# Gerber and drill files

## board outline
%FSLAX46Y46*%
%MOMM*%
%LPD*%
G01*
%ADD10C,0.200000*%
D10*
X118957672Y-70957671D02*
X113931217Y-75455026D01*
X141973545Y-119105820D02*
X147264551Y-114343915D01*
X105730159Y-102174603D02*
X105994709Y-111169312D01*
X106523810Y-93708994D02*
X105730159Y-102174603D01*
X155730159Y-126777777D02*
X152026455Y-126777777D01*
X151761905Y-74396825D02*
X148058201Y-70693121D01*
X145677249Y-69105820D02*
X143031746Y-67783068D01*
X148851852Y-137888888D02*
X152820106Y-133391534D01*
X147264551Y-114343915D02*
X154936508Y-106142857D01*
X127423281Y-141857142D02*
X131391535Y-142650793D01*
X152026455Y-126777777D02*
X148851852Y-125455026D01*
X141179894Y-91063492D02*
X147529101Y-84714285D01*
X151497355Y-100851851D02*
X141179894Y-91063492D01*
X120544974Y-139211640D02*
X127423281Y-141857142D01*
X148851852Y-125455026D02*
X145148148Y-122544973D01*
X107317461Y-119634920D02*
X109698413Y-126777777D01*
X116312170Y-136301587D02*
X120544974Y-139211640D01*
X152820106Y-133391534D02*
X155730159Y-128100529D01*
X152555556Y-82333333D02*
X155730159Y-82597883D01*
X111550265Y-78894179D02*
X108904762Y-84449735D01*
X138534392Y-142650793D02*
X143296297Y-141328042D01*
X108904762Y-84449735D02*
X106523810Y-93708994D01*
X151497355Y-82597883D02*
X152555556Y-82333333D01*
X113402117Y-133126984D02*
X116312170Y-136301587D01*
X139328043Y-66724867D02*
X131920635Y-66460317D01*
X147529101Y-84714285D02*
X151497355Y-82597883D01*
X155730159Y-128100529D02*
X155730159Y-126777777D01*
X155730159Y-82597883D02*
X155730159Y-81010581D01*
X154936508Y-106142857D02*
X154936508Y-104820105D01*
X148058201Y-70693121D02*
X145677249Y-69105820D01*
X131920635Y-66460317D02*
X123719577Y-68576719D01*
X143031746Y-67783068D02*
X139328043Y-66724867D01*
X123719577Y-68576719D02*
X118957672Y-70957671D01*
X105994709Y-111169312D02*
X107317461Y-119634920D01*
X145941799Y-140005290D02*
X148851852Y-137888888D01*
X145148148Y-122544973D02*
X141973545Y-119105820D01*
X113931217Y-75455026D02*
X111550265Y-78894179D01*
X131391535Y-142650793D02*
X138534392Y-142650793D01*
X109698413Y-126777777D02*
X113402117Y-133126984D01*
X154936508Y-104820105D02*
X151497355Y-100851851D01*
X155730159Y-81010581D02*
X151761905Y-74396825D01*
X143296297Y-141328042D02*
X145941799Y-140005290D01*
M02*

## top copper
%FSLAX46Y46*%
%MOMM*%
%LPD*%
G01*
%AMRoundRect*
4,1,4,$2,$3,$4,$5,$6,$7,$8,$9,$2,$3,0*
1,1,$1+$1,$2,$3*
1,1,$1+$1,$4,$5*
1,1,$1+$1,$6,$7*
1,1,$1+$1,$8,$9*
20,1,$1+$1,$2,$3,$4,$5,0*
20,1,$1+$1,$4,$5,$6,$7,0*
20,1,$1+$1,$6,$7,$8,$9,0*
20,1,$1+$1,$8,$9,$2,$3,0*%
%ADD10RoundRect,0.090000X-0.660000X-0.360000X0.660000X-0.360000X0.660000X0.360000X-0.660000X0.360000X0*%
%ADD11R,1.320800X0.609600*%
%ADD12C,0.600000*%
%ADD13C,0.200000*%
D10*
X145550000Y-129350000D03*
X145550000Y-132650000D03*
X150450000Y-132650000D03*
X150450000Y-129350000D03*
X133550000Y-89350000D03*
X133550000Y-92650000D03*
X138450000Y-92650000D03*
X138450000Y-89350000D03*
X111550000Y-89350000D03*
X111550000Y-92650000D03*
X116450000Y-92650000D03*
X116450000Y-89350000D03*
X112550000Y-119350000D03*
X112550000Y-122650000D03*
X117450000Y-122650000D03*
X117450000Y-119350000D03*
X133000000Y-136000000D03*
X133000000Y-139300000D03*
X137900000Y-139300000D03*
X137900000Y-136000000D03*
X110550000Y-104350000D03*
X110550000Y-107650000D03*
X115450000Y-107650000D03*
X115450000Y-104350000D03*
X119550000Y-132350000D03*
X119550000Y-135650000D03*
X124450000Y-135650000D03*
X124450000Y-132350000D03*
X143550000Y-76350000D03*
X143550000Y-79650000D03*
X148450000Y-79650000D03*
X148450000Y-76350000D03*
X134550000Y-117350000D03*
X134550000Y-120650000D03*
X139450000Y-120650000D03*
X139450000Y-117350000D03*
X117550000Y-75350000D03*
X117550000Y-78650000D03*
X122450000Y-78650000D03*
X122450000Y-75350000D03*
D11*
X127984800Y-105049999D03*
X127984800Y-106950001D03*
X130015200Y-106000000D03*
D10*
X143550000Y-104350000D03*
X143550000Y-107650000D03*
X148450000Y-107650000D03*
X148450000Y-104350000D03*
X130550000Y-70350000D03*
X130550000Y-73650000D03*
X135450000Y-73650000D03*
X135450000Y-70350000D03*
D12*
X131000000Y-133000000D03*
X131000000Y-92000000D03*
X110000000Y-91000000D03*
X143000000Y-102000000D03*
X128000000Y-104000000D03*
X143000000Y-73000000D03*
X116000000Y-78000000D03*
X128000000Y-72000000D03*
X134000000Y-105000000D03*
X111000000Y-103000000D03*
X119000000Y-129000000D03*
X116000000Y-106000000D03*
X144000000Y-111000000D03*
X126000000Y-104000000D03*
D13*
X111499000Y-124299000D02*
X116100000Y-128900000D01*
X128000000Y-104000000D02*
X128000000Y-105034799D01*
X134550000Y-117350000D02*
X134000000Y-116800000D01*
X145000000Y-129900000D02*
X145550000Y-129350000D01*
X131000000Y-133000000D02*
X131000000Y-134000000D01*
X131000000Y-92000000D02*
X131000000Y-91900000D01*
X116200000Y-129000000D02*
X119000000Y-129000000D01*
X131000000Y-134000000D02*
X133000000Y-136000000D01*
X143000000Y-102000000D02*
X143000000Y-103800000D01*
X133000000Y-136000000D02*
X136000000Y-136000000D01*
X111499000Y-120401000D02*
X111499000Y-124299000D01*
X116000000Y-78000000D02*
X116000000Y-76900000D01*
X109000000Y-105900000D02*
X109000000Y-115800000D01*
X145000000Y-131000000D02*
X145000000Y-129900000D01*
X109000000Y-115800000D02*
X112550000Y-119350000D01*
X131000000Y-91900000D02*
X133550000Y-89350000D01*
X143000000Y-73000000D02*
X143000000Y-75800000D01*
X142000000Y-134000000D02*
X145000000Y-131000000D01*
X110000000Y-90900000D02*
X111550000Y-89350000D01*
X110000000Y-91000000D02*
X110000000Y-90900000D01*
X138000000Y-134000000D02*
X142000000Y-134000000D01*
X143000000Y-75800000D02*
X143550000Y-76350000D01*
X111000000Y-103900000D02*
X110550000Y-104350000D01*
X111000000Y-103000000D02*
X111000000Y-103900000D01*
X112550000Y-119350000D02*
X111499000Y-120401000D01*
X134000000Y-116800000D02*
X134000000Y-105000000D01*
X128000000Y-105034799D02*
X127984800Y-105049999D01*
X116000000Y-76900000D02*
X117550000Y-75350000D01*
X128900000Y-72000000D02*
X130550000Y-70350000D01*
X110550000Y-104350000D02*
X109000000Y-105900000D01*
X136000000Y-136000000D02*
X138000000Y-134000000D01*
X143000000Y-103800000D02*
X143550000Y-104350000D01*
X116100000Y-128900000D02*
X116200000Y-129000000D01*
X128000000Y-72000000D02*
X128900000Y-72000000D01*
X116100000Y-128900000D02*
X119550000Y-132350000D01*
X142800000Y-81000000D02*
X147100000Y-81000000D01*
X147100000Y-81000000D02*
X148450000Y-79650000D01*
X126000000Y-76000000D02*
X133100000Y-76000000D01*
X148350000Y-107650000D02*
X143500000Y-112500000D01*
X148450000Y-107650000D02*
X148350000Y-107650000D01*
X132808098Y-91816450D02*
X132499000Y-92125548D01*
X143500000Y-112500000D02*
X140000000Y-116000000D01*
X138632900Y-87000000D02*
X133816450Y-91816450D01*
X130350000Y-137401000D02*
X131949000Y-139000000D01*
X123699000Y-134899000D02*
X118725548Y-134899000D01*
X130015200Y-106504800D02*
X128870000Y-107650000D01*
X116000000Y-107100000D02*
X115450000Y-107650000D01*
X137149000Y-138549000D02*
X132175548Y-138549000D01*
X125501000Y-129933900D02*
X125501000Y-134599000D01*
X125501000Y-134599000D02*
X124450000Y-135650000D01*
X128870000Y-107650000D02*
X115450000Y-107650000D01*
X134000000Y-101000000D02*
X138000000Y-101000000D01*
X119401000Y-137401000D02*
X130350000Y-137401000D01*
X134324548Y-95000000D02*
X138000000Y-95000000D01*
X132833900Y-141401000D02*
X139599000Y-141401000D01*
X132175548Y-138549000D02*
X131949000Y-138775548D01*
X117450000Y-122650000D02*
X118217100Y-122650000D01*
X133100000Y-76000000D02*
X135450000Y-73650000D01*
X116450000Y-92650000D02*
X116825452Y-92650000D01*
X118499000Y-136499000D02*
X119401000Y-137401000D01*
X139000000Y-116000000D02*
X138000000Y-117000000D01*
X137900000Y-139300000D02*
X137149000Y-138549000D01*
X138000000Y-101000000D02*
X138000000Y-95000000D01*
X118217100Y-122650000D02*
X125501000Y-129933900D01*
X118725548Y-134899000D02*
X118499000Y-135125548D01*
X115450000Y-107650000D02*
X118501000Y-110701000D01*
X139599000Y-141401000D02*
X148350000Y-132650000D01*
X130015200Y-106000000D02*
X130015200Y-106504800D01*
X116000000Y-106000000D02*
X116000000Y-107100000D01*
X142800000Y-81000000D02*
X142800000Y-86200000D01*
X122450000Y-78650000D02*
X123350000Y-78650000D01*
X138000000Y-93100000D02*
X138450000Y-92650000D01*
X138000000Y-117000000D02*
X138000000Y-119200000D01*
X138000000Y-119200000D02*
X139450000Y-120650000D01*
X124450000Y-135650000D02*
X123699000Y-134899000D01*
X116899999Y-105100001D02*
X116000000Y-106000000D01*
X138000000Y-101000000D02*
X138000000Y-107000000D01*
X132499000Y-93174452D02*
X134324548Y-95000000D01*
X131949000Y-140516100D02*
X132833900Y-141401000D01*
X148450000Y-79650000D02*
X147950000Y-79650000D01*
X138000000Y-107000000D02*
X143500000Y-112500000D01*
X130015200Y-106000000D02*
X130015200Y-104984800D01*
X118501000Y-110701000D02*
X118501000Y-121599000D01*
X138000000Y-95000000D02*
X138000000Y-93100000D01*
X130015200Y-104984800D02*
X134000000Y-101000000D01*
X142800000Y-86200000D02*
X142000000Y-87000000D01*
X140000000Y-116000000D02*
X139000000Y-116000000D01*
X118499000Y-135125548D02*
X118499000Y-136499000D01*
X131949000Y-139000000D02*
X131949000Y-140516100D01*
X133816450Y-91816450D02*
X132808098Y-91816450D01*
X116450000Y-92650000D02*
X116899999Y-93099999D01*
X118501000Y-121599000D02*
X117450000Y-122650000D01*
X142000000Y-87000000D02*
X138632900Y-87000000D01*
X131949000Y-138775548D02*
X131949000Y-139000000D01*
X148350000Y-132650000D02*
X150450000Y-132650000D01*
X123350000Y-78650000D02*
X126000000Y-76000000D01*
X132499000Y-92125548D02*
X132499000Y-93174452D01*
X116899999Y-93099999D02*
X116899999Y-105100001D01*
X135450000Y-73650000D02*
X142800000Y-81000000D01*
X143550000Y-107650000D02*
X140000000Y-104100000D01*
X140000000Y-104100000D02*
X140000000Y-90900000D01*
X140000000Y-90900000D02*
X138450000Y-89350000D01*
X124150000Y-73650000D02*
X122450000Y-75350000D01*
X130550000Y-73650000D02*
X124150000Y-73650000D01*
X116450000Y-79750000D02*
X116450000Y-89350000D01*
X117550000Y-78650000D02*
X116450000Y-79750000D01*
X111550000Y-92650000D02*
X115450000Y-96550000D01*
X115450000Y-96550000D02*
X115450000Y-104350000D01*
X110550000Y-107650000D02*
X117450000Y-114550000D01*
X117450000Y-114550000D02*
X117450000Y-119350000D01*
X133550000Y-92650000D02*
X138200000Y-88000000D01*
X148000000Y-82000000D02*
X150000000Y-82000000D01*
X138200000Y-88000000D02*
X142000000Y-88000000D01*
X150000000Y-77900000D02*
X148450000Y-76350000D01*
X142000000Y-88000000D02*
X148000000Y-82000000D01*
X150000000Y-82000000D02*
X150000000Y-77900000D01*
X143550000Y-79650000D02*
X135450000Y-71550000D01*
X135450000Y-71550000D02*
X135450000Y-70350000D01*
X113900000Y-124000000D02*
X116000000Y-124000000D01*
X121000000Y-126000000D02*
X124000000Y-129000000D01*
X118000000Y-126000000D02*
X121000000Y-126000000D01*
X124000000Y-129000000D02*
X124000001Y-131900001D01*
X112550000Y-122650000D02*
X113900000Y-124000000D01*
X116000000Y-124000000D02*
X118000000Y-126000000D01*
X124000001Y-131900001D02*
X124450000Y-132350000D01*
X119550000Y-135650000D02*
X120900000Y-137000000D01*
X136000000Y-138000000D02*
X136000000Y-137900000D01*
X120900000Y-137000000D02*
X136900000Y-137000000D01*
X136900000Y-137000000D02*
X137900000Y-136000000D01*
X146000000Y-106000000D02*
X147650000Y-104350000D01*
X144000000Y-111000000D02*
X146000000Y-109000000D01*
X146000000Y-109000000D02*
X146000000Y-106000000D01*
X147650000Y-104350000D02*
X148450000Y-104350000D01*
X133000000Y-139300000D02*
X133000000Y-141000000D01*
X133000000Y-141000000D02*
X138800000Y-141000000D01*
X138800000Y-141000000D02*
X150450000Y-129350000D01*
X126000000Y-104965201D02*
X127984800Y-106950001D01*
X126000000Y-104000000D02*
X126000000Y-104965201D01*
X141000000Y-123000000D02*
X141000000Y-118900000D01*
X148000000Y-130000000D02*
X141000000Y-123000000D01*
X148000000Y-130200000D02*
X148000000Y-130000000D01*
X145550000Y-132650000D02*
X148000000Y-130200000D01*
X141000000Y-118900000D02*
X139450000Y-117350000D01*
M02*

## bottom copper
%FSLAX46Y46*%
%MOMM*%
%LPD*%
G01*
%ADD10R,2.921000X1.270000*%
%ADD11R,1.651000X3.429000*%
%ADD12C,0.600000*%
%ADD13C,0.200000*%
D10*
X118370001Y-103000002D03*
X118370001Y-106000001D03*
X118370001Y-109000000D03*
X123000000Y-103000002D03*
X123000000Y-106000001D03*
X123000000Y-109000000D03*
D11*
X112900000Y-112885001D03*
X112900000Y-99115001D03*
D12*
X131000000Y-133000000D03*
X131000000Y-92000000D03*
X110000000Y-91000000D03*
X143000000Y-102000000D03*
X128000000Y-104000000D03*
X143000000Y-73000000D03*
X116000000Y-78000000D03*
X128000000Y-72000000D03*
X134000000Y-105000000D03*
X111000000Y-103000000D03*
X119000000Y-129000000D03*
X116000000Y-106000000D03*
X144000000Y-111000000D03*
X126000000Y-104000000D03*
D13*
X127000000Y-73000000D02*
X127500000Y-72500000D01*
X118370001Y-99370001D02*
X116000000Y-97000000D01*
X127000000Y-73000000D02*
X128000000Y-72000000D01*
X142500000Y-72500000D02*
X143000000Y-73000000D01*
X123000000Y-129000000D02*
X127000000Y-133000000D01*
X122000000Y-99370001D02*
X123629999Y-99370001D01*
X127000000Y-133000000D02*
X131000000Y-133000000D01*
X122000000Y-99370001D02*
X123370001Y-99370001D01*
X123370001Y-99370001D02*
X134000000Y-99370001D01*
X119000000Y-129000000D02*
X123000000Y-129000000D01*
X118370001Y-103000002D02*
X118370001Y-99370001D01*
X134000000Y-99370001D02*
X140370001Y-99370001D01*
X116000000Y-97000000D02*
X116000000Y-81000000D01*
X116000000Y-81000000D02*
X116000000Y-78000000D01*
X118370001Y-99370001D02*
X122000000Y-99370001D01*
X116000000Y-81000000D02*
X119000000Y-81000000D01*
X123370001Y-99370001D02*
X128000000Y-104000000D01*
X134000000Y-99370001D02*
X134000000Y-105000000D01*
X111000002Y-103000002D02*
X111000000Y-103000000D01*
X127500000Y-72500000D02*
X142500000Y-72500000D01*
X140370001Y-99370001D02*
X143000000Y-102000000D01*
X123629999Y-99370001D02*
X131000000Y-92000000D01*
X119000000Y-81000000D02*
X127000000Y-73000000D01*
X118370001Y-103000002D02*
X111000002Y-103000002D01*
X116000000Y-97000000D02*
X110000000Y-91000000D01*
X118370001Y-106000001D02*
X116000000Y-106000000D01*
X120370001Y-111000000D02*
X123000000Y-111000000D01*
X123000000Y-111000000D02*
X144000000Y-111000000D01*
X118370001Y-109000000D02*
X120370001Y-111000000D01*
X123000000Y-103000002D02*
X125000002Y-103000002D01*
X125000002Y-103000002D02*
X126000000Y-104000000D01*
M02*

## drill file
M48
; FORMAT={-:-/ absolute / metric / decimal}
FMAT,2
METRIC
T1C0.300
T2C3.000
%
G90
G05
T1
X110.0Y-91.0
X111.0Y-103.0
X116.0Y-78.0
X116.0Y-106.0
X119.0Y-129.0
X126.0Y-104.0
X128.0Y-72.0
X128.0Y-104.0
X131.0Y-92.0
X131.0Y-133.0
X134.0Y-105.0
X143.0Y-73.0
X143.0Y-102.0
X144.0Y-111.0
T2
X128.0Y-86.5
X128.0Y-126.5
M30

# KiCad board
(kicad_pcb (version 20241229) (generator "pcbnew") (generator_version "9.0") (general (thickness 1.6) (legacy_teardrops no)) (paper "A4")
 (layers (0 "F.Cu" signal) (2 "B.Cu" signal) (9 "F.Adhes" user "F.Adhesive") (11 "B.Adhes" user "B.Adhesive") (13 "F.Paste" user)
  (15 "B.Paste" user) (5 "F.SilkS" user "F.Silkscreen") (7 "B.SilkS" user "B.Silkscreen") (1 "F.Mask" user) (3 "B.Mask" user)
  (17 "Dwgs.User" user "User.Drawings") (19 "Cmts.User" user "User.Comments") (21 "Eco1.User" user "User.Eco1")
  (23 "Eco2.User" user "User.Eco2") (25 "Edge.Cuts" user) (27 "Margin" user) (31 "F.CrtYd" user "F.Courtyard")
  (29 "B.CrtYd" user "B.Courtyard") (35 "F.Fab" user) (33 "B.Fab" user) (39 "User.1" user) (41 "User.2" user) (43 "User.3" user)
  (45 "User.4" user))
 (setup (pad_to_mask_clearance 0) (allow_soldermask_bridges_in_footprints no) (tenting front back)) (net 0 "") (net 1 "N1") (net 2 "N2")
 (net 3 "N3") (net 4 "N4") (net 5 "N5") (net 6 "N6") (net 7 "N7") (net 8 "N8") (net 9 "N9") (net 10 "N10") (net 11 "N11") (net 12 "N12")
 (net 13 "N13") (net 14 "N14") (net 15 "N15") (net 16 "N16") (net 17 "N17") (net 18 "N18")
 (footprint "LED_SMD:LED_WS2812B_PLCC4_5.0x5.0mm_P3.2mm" (layer "F.Cu") (at 148 131)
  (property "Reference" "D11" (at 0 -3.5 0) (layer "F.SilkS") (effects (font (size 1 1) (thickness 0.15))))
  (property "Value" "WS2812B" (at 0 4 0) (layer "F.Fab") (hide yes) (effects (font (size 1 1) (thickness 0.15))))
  (pad "1" smd roundrect (at -2.45 -1.65) (size 1.5 0.9) (layers "F.Cu" "F.Mask" "F.Paste") (roundrect_rratio 0.1) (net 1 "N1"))
  (pad "2" smd roundrect (at -2.45 1.65) (size 1.5 0.9) (layers "F.Cu" "F.Mask" "F.Paste") (roundrect_rratio 0.1) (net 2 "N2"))
  (pad "3" smd roundrect (at 2.45 1.65) (size 1.5 0.9) (layers "F.Cu" "F.Mask" "F.Paste") (roundrect_rratio 0.1) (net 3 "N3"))
  (pad "4" smd roundrect (at 2.45 -1.65) (size 1.5 0.9) (layers "F.Cu" "F.Mask" "F.Paste") (roundrect_rratio 0.1) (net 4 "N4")))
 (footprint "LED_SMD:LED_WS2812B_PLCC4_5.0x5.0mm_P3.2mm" (layer "F.Cu") (at 136 91)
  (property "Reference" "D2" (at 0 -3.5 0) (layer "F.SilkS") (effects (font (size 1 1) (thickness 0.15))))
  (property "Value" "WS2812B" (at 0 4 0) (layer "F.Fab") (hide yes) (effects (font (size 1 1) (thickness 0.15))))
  (pad "1" smd roundrect (at -2.45 -1.65) (size 1.5 0.9) (layers "F.Cu" "F.Mask" "F.Paste") (roundrect_rratio 0.1) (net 1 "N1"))
  (pad "2" smd roundrect (at -2.45 1.65) (size 1.5 0.9) (layers "F.Cu" "F.Mask" "F.Paste") (roundrect_rratio 0.1) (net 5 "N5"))
  (pad "3" smd roundrect (at 2.45 1.65) (size 1.5 0.9) (layers "F.Cu" "F.Mask" "F.Paste") (roundrect_rratio 0.1) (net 3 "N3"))
  (pad "4" smd roundrect (at 2.45 -1.65) (size 1.5 0.9) (layers "F.Cu" "F.Mask" "F.Paste") (roundrect_rratio 0.1) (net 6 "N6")))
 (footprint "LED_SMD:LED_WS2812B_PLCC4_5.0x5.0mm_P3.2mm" (layer "F.Cu") (at 114 91)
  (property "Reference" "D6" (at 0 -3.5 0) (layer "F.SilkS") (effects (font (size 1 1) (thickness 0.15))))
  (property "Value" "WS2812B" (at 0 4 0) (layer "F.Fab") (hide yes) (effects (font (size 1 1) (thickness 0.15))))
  (pad "1" smd roundrect (at -2.45 -1.65) (size 1.5 0.9) (layers "F.Cu" "F.Mask" "F.Paste") (roundrect_rratio 0.1) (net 1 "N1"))
  (pad "2" smd roundrect (at -2.45 1.65) (size 1.5 0.9) (layers "F.Cu" "F.Mask" "F.Paste") (roundrect_rratio 0.1) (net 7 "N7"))
  (pad "3" smd roundrect (at 2.45 1.65) (size 1.5 0.9) (layers "F.Cu" "F.Mask" "F.Paste") (roundrect_rratio 0.1) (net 3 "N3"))
  (pad "4" smd roundrect (at 2.45 -1.65) (size 1.5 0.9) (layers "F.Cu" "F.Mask" "F.Paste") (roundrect_rratio 0.1) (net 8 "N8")))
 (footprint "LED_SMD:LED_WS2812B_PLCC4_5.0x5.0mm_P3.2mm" (layer "F.Cu") (at 115 121)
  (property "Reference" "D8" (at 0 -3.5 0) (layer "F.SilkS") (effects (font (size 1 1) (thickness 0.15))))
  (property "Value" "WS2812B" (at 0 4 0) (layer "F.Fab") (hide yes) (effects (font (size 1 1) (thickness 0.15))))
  (pad "1" smd roundrect (at -2.45 -1.65) (size 1.5 0.9) (layers "F.Cu" "F.Mask" "F.Paste") (roundrect_rratio 0.1) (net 1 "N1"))
  (pad "2" smd roundrect (at -2.45 1.65) (size 1.5 0.9) (layers "F.Cu" "F.Mask" "F.Paste") (roundrect_rratio 0.1) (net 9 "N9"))
  (pad "3" smd roundrect (at 2.45 1.65) (size 1.5 0.9) (layers "F.Cu" "F.Mask" "F.Paste") (roundrect_rratio 0.1) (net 3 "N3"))
  (pad "4" smd roundrect (at 2.45 -1.65) (size 1.5 0.9) (layers "F.Cu" "F.Mask" "F.Paste") (roundrect_rratio 0.1) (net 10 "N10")))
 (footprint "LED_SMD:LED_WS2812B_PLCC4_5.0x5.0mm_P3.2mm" (layer "F.Cu") (at 135.45 137.65)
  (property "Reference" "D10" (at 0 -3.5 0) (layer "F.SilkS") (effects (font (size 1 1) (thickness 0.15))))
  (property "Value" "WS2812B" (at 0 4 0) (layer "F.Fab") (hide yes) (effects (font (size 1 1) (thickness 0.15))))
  (pad "1" smd roundrect (at -2.45 -1.65) (size 1.5 0.9) (layers "F.Cu" "F.Mask" "F.Paste") (roundrect_rratio 0.1) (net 1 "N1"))
  (pad "2" smd roundrect (at -2.45 1.65) (size 1.5 0.9) (layers "F.Cu" "F.Mask" "F.Paste") (roundrect_rratio 0.1) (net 4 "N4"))
  (pad "3" smd roundrect (at 2.45 1.65) (size 1.5 0.9) (layers "F.Cu" "F.Mask" "F.Paste") (roundrect_rratio 0.1) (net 3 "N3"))
  (pad "4" smd roundrect (at 2.45 -1.65) (size 1.5 0.9) (layers "F.Cu" "F.Mask" "F.Paste") (roundrect_rratio 0.1) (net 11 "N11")))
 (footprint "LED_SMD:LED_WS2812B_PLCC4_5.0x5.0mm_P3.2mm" (layer "F.Cu") (at 113 106)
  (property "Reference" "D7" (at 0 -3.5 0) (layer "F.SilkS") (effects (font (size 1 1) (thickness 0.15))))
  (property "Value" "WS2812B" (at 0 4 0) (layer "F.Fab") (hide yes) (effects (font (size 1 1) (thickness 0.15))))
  (pad "1" smd roundrect (at -2.45 -1.65) (size 1.5 0.9) (layers "F.Cu" "F.Mask" "F.Paste") (roundrect_rratio 0.1) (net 1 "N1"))
  (pad "2" smd roundrect (at -2.45 1.65) (size 1.5 0.9) (layers "F.Cu" "F.Mask" "F.Paste") (roundrect_rratio 0.1) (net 10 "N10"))
  (pad "3" smd roundrect (at 2.45 1.65) (size 1.5 0.9) (layers "F.Cu" "F.Mask" "F.Paste") (roundrect_rratio 0.1) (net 3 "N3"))
  (pad "4" smd roundrect (at 2.45 -1.65) (size 1.5 0.9) (layers "F.Cu" "F.Mask" "F.Paste") (roundrect_rratio 0.1) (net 7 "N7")))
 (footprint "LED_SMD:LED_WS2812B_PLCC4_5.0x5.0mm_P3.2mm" (layer "F.Cu") (at 122 134)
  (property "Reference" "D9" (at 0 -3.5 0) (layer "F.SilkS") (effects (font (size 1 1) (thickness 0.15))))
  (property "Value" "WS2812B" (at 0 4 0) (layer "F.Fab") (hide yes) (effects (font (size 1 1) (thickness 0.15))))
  (pad "1" smd roundrect (at -2.45 -1.65) (size 1.5 0.9) (layers "F.Cu" "F.Mask" "F.Paste") (roundrect_rratio 0.1) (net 1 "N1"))
  (pad "2" smd roundrect (at -2.45 1.65) (size 1.5 0.9) (layers "F.Cu" "F.Mask" "F.Paste") (roundrect_rratio 0.1) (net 11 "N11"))
  (pad "3" smd roundrect (at 2.45 1.65) (size 1.5 0.9) (layers "F.Cu" "F.Mask" "F.Paste") (roundrect_rratio 0.1) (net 3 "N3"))
  (pad "4" smd roundrect (at 2.45 -1.65) (size 1.5 0.9) (layers "F.Cu" "F.Mask" "F.Paste") (roundrect_rratio 0.1) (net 9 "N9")))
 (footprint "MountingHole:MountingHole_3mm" (layer "F.Cu") (at 128 126.5)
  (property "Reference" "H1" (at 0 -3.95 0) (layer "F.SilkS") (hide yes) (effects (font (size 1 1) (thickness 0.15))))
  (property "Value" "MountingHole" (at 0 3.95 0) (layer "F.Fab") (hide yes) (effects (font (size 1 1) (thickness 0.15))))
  (pad "" np_thru_hole circle (at 0 0) (size 3 3) (drill 3) (layers "*.Cu" "*.Mask")))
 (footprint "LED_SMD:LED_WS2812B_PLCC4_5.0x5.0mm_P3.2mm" (layer "F.Cu") (at 146 78)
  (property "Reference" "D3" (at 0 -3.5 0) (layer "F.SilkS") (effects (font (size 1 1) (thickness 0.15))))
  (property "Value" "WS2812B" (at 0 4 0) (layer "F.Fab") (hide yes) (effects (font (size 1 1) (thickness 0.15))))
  (pad "1" smd roundrect (at -2.45 -1.65) (size 1.5 0.9) (layers "F.Cu" "F.Mask" "F.Paste") (roundrect_rratio 0.1) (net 1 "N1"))
  (pad "2" smd roundrect (at -2.45 1.65) (size 1.5 0.9) (layers "F.Cu" "F.Mask" "F.Paste") (roundrect_rratio 0.1) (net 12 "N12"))
  (pad "3" smd roundrect (at 2.45 1.65) (size 1.5 0.9) (layers "F.Cu" "F.Mask" "F.Paste") (roundrect_rratio 0.1) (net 3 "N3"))
  (pad "4" smd roundrect (at 2.45 -1.65) (size 1.5 0.9) (layers "F.Cu" "F.Mask" "F.Paste") (roundrect_rratio 0.1) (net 5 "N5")))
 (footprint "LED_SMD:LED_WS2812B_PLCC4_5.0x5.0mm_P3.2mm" (layer "F.Cu") (at 137 119)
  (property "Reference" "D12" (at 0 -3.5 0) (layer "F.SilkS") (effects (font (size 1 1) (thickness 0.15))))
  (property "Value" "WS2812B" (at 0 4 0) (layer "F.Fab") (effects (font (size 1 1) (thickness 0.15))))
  (pad "1" smd roundrect (at -2.45 -1.65) (size 1.5 0.9) (layers "F.Cu" "F.Mask" "F.Paste") (roundrect_rratio 0.1) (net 1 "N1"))
  (pad "2" smd roundrect (at -2.45 1.65) (size 1.5 0.9) (layers "F.Cu" "F.Mask" "F.Paste") (roundrect_rratio 0.1) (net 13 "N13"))
  (pad "3" smd roundrect (at 2.45 1.65) (size 1.5 0.9) (layers "F.Cu" "F.Mask" "F.Paste") (roundrect_rratio 0.1) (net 3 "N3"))
  (pad "4" smd roundrect (at 2.45 -1.65) (size 1.5 0.9) (layers "F.Cu" "F.Mask" "F.Paste") (roundrect_rratio 0.1) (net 2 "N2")))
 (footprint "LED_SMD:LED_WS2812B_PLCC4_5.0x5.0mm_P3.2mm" (layer "F.Cu") (at 120 77)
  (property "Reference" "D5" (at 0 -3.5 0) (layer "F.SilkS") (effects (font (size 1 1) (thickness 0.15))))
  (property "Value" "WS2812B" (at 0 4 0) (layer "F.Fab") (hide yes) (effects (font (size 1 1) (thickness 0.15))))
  (pad "1" smd roundrect (at -2.45 -1.65) (size 1.5 0.9) (layers "F.Cu" "F.Mask" "F.Paste") (roundrect_rratio 0.1) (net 1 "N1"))
  (pad "2" smd roundrect (at -2.45 1.65) (size 1.5 0.9) (layers "F.Cu" "F.Mask" "F.Paste") (roundrect_rratio 0.1) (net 8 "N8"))
  (pad "3" smd roundrect (at 2.45 1.65) (size 1.5 0.9) (layers "F.Cu" "F.Mask" "F.Paste") (roundrect_rratio 0.1) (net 3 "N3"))
  (pad "4" smd roundrect (at 2.45 -1.65) (size 1.5 0.9) (layers "F.Cu" "F.Mask" "F.Paste") (roundrect_rratio 0.1) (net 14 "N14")))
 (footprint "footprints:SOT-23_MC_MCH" (layer "F.Cu") (at 129 106 -90)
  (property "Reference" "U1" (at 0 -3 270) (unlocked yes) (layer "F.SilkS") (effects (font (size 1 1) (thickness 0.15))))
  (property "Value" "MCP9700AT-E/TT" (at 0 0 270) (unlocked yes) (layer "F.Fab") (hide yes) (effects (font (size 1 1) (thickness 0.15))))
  (pad "1" smd rect (at -0.950001 1.0152 270) (size 0.6096 1.3208) (layers "F.Cu" "F.Mask" "F.Paste") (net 1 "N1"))
  (pad "2" smd rect (at 0.950001 1.0152 270) (size 0.6096 1.3208) (layers "F.Cu" "F.Mask" "F.Paste") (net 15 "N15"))
  (pad "3" smd rect (at 0 -1.0152 270) (size 0.6096 1.3208) (layers "F.Cu" "F.Mask" "F.Paste") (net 3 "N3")))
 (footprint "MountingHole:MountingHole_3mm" (layer "F.Cu") (at 128 86.5)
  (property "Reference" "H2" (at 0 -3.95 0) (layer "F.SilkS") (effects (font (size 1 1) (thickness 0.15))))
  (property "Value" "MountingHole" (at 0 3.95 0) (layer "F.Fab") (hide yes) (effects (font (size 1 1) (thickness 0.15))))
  (pad "" np_thru_hole circle (at 0 0) (size 3 3) (drill 3) (layers "*.Cu" "*.Mask")))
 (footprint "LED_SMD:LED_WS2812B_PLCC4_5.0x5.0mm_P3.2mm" (layer "F.Cu") (at 146 106)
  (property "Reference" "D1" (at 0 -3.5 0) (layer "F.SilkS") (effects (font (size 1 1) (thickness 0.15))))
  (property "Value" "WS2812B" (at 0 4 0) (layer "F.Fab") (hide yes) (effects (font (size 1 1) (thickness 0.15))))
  (pad "1" smd roundrect (at -2.45 -1.65) (size 1.5 0.9) (layers "F.Cu" "F.Mask" "F.Paste") (roundrect_rratio 0.1) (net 1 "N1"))
  (pad "2" smd roundrect (at -2.45 1.65) (size 1.5 0.9) (layers "F.Cu" "F.Mask" "F.Paste") (roundrect_rratio 0.1) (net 6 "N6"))
  (pad "3" smd roundrect (at 2.45 1.65) (size 1.5 0.9) (layers "F.Cu" "F.Mask" "F.Paste") (roundrect_rratio 0.1) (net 3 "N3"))
  (pad "4" smd roundrect (at 2.45 -1.65) (size 1.5 0.9) (layers "F.Cu" "F.Mask" "F.Paste") (roundrect_rratio 0.1) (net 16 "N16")))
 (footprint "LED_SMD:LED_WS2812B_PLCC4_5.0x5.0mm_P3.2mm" (layer "F.Cu") (at 133 72)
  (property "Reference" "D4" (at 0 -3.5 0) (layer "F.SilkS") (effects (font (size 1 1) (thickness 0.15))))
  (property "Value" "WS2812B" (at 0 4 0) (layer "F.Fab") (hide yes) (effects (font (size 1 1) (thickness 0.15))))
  (pad "1" smd roundrect (at -2.45 -1.65) (size 1.5 0.9) (layers "F.Cu" "F.Mask" "F.Paste") (roundrect_rratio 0.1) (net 1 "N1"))
  (pad "2" smd roundrect (at -2.45 1.65) (size 1.5 0.9) (layers "F.Cu" "F.Mask" "F.Paste") (roundrect_rratio 0.1) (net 14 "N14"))
  (pad "3" smd roundrect (at 2.45 1.65) (size 1.5 0.9) (layers "F.Cu" "F.Mask" "F.Paste") (roundrect_rratio 0.1) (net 3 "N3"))
  (pad "4" smd roundrect (at 2.45 -1.65) (size 1.5 0.9) (layers "F.Cu" "F.Mask" "F.Paste") (roundrect_rratio 0.1) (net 12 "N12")))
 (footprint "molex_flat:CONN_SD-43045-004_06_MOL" (layer "B.Cu") (at 113.257002 106.000001 90)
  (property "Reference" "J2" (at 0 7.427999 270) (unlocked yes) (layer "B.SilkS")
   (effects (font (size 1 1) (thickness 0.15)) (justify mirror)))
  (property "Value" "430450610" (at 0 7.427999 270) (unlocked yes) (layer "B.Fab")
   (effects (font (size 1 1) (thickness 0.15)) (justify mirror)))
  (pad "1" smd rect (at 2.999999 5.112999 90) (size 1.27 2.921) (layers "B.Cu" "B.Mask" "B.Paste") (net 1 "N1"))
  (pad "2" smd rect (at 0 5.112999 90) (size 1.27 2.921) (layers "B.Cu" "B.Mask" "B.Paste") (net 3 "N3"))
  (pad "3" smd rect (at -2.999999 5.112999 90) (size 1.27 2.921) (layers "B.Cu" "B.Mask" "B.Paste") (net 16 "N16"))
  (pad "4" smd rect (at 2.999999 9.742998 90) (size 1.27 2.921) (layers "B.Cu" "B.Mask" "B.Paste") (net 15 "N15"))
  (pad "5" smd rect (at 0 9.742998 90) (size 1.27 2.921) (layers "B.Cu" "B.Mask" "B.Paste") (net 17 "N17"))
  (pad "6" smd rect (at -2.999999 9.742998 90) (size 1.27 2.921) (layers "B.Cu" "B.Mask" "B.Paste") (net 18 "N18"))
  (pad "7" smd rect (at -6.885 -0.357002 90) (size 3.429 1.651) (layers "B.Cu" "B.Mask" "B.Paste"))
  (pad "8" smd rect (at 6.885 -0.357002 90) (size 3.429 1.651) (layers "B.Cu" "B.Mask" "B.Paste")))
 (gr_line (start 118.957672 70.957671) (end 113.931217 75.455026) (stroke (width 0.2) (type default)) (layer "Edge.Cuts"))
 (gr_line (start 141.973545 119.10582) (end 147.264551 114.343915) (stroke (width 0.2) (type default)) (layer "Edge.Cuts"))
 (gr_line (start 105.730159 102.174603) (end 105.994709 111.169312) (stroke (width 0.2) (type default)) (layer "Edge.Cuts"))
 (gr_line (start 106.52381 93.708994) (end 105.730159 102.174603) (stroke (width 0.2) (type default)) (layer "Edge.Cuts"))
 (gr_line (start 155.730159 126.777777) (end 152.026455 126.777777) (stroke (width 0.2) (type default)) (layer "Edge.Cuts"))
 (gr_line (start 151.761905 74.396825) (end 148.058201 70.693121) (stroke (width 0.2) (type default)) (layer "Edge.Cuts"))
 (gr_line (start 145.677249 69.10582) (end 143.031746 67.783068) (stroke (width 0.2) (type default)) (layer "Edge.Cuts"))
 (gr_line (start 148.851852 137.888888) (end 152.820106 133.391534) (stroke (width 0.2) (type default)) (layer "Edge.Cuts"))
 (gr_line (start 147.264551 114.343915) (end 154.936508 106.142857) (stroke (width 0.2) (type default)) (layer "Edge.Cuts"))
 (gr_line (start 127.423281 141.857142) (end 131.391535 142.650793) (stroke (width 0.2) (type default)) (layer "Edge.Cuts"))
 (gr_line (start 152.026455 126.777777) (end 148.851852 125.455026) (stroke (width 0.2) (type default)) (layer "Edge.Cuts"))
 (gr_line (start 141.179894 91.063492) (end 147.529101 84.714285) (stroke (width 0.2) (type default)) (layer "Edge.Cuts"))
 (gr_line (start 151.497355 100.851851) (end 141.179894 91.063492) (stroke (width 0.2) (type default)) (layer "Edge.Cuts"))
 (gr_line (start 120.544974 139.21164) (end 127.423281 141.857142) (stroke (width 0.2) (type default)) (layer "Edge.Cuts"))
 (gr_line (start 148.851852 125.455026) (end 145.148148 122.544973) (stroke (width 0.2) (type default)) (layer "Edge.Cuts"))
 (gr_line (start 107.317461 119.63492) (end 109.698413 126.777777) (stroke (width 0.2) (type default)) (layer "Edge.Cuts"))
 (gr_line (start 116.31217 136.301587) (end 120.544974 139.21164) (stroke (width 0.2) (type default)) (layer "Edge.Cuts"))
 (gr_line (start 152.820106 133.391534) (end 155.730159 128.100529) (stroke (width 0.2) (type default)) (layer "Edge.Cuts"))
 (gr_line (start 152.555556 82.333333) (end 155.730159 82.597883) (stroke (width 0.2) (type default)) (layer "Edge.Cuts"))
 (gr_line (start 111.550265 78.894179) (end 108.904762 84.449735) (stroke (width 0.2) (type default)) (layer "Edge.Cuts"))
 (gr_line (start 138.534392 142.650793) (end 143.296297 141.328042) (stroke (width 0.2) (type default)) (layer "Edge.Cuts"))
 (gr_line (start 108.904762 84.449735) (end 106.52381 93.708994) (stroke (width 0.2) (type default)) (layer "Edge.Cuts"))
 (gr_line (start 151.497355 82.597883) (end 152.555556 82.333333) (stroke (width 0.2) (type default)) (layer "Edge.Cuts"))
 (gr_line (start 113.402117 133.126984) (end 116.31217 136.301587) (stroke (width 0.2) (type default)) (layer "Edge.Cuts"))
 (gr_line (start 139.328043 66.724867) (end 131.920635 66.460317) (stroke (width 0.2) (type default)) (layer "Edge.Cuts"))
 (gr_line (start 147.529101 84.714285) (end 151.497355 82.597883) (stroke (width 0.2) (type default)) (layer "Edge.Cuts"))
 (gr_line (start 155.730159 128.100529) (end 155.730159 126.777777) (stroke (width 0.2) (type default)) (layer "Edge.Cuts"))
 (gr_line (start 155.730159 82.597883) (end 155.730159 81.010581) (stroke (width 0.2) (type default)) (layer "Edge.Cuts"))
 (gr_line (start 154.936508 106.142857) (end 154.936508 104.820105) (stroke (width 0.2) (type default)) (layer "Edge.Cuts"))
 (gr_line (start 148.058201 70.693121) (end 145.677249 69.10582) (stroke (width 0.2) (type default)) (layer "Edge.Cuts"))
 (gr_line (start 131.920635 66.460317) (end 123.719577 68.576719) (stroke (width 0.2) (type default)) (layer "Edge.Cuts"))
 (gr_line (start 143.031746 67.783068) (end 139.328043 66.724867) (stroke (width 0.2) (type default)) (layer "Edge.Cuts"))
 (gr_line (start 123.719577 68.576719) (end 118.957672 70.957671) (stroke (width 0.2) (type default)) (layer "Edge.Cuts"))
 (gr_line (start 105.994709 111.169312) (end 107.317461 119.63492) (stroke (width 0.2) (type default)) (layer "Edge.Cuts"))
 (gr_line (start 145.941799 140.00529) (end 148.851852 137.888888) (stroke (width 0.2) (type default)) (layer "Edge.Cuts"))
 (gr_line (start 145.148148 122.544973) (end 141.973545 119.10582) (stroke (width 0.2) (type default)) (layer "Edge.Cuts"))
 (gr_line (start 113.931217 75.455026) (end 111.550265 78.894179) (stroke (width 0.2) (type default)) (layer "Edge.Cuts"))
 (gr_line (start 131.391535 142.650793) (end 138.534392 142.650793) (stroke (width 0.2) (type default)) (layer "Edge.Cuts"))
 (gr_line (start 109.698413 126.777777) (end 113.402117 133.126984) (stroke (width 0.2) (type default)) (layer "Edge.Cuts"))
 (gr_line (start 154.936508 104.820105) (end 151.497355 100.851851) (stroke (width 0.2) (type default)) (layer "Edge.Cuts"))
 (gr_line (start 155.730159 81.010581) (end 151.761905 74.396825) (stroke (width 0.2) (type default)) (layer "Edge.Cuts"))
 (gr_line (start 143.296297 141.328042) (end 145.941799 140.00529) (stroke (width 0.2) (type default)) (layer "Edge.Cuts"))
 (segment (start 111.499 124.299) (end 116.1 128.9) (width 0.2) (layer "F.Cu") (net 1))
 (segment (start 128 104) (end 128 105.034799) (width 0.2) (layer "F.Cu") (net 1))
 (segment (start 134.55 117.35) (end 134 116.8) (width 0.2) (layer "F.Cu") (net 1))
 (segment (start 145 129.9) (end 145.55 129.35) (width 0.2) (layer "F.Cu") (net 1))
 (segment (start 131 133) (end 131 134) (width 0.2) (layer "F.Cu") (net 1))
 (segment (start 131 92) (end 131 91.9) (width 0.2) (layer "F.Cu") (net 1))
 (segment (start 116.2 129) (end 119 129) (width 0.2) (layer "F.Cu") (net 1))
 (segment (start 131 134) (end 133 136) (width 0.2) (layer "F.Cu") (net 1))
 (segment (start 143 102) (end 143 103.8) (width 0.2) (layer "F.Cu") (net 1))
 (segment (start 133 136) (end 136 136) (width 0.2) (layer "F.Cu") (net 1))
 (segment (start 111.499 120.401) (end 111.499 124.299) (width 0.2) (layer "F.Cu") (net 1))
 (segment (start 116 78) (end 116 76.9) (width 0.2) (layer "F.Cu") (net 1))
 (segment (start 109 105.9) (end 109 115.8) (width 0.2) (layer "F.Cu") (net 1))
 (segment (start 145 131) (end 145 129.9) (width 0.2) (layer "F.Cu") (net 1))
 (segment (start 109 115.8) (end 112.55 119.35) (width 0.2) (layer "F.Cu") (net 1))
 (segment (start 131 91.9) (end 133.55 89.35) (width 0.2) (layer "F.Cu") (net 1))
 (segment (start 143 73) (end 143 75.8) (width 0.2) (layer "F.Cu") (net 1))
 (segment (start 142 134) (end 145 131) (width 0.2) (layer "F.Cu") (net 1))
 (segment (start 110 90.9) (end 111.55 89.35) (width 0.2) (layer "F.Cu") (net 1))
 (segment (start 110 91) (end 110 90.9) (width 0.2) (layer "F.Cu") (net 1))
 (segment (start 138 134) (end 142 134) (width 0.2) (layer "F.Cu") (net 1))
 (segment (start 143 75.8) (end 143.55 76.35) (width 0.2) (layer "F.Cu") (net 1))
 (segment (start 111 103.9) (end 110.55 104.35) (width 0.2) (layer "F.Cu") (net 1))
 (segment (start 111 103) (end 111 103.9) (width 0.2) (layer "F.Cu") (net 1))
 (segment (start 112.55 119.35) (end 111.499 120.401) (width 0.2) (layer "F.Cu") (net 1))
 (segment (start 134 116.8) (end 134 105) (width 0.2) (layer "F.Cu") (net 1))
 (segment (start 128 105.034799) (end 127.9848 105.049999) (width 0.2) (layer "F.Cu") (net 1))
 (segment (start 116 76.9) (end 117.55 75.35) (width 0.2) (layer "F.Cu") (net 1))
 (segment (start 128.9 72) (end 130.55 70.35) (width 0.2) (layer "F.Cu") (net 1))
 (segment (start 110.55 104.35) (end 109 105.9) (width 0.2) (layer "F.Cu") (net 1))
 (segment (start 136 136) (end 138 134) (width 0.2) (layer "F.Cu") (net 1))
 (segment (start 143 103.8) (end 143.55 104.35) (width 0.2) (layer "F.Cu") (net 1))
 (segment (start 116.1 128.9) (end 116.2 129) (width 0.2) (layer "F.Cu") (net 1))
 (segment (start 128 72) (end 128.9 72) (width 0.2) (layer "F.Cu") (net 1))
 (segment (start 116.1 128.9) (end 119.55 132.35) (width 0.2) (layer "F.Cu") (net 1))
 (via (at 131 133) (size 0.6) (drill 0.3) (layers "F.Cu" "B.Cu") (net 1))
 (via (at 131 92) (size 0.6) (drill 0.3) (layers "F.Cu" "B.Cu") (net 1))
 (via (at 110 91) (size 0.6) (drill 0.3) (layers "F.Cu" "B.Cu") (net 1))
 (via (at 143 102) (size 0.6) (drill 0.3) (layers "F.Cu" "B.Cu") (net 1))
 (via (at 128 104) (size 0.6) (drill 0.3) (layers "F.Cu" "B.Cu") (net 1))
 (via (at 143 73) (size 0.6) (drill 0.3) (layers "F.Cu" "B.Cu") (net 1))
 (via (at 116 78) (size 0.6) (drill 0.3) (layers "F.Cu" "B.Cu") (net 1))
 (via (at 128 72) (size 0.6) (drill 0.3) (layers "F.Cu" "B.Cu") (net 1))
 (via (at 134 105) (size 0.6) (drill 0.3) (layers "F.Cu" "B.Cu") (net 1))
 (via (at 111 103) (size 0.6) (drill 0.3) (layers "F.Cu" "B.Cu") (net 1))
 (via (at 119 129) (size 0.6) (drill 0.3) (layers "F.Cu" "B.Cu") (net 1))
 (segment (start 127 73) (end 127.5 72.5) (width 0.2) (layer "B.Cu") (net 1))
 (segment (start 118.370001 99.370001) (end 116 97) (width 0.2) (layer "B.Cu") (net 1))
 (segment (start 127 73) (end 128 72) (width 0.2) (layer "B.Cu") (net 1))
 (segment (start 142.5 72.5) (end 143 73) (width 0.2) (layer "B.Cu") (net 1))
 (segment (start 123 129) (end 127 133) (width 0.2) (layer "B.Cu") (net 1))
 (segment (start 122 99.370001) (end 123.629999 99.370001) (width 0.2) (layer "B.Cu") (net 1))
 (segment (start 127 133) (end 131 133) (width 0.2) (layer "B.Cu") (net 1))
 (segment (start 122 99.370001) (end 123.370001 99.370001) (width 0.2) (layer "B.Cu") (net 1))
 (segment (start 123.370001 99.370001) (end 134 99.370001) (width 0.2) (layer "B.Cu") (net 1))
 (segment (start 119 129) (end 123 129) (width 0.2) (layer "B.Cu") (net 1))
 (segment (start 118.370001 103.000002) (end 118.370001 99.370001) (width 0.2) (layer "B.Cu") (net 1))
 (segment (start 134 99.370001) (end 140.370001 99.370001) (width 0.2) (layer "B.Cu") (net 1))
 (segment (start 116 97) (end 116 81) (width 0.2) (layer "B.Cu") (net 1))
 (segment (start 116 81) (end 116 78) (width 0.2) (layer "B.Cu") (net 1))
 (segment (start 118.370001 99.370001) (end 122 99.370001) (width 0.2) (layer "B.Cu") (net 1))
 (segment (start 116 81) (end 119 81) (width 0.2) (layer "B.Cu") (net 1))
 (segment (start 123.370001 99.370001) (end 128 104) (width 0.2) (layer "B.Cu") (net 1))
 (segment (start 134 99.370001) (end 134 105) (width 0.2) (layer "B.Cu") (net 1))
 (segment (start 111.000002 103.000002) (end 111 103) (width 0.2) (layer "B.Cu") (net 1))
 (segment (start 127.5 72.5) (end 142.5 72.5) (width 0.2) (layer "B.Cu") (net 1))
 (segment (start 140.370001 99.370001) (end 143 102) (width 0.2) (layer "B.Cu") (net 1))
 (segment (start 123.629999 99.370001) (end 131 92) (width 0.2) (layer "B.Cu") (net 1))
 (segment (start 119 81) (end 127 73) (width 0.2) (layer "B.Cu") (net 1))
 (segment (start 118.370001 103.000002) (end 111.000002 103.000002) (width 0.2) (layer "B.Cu") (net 1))
 (segment (start 116 97) (end 110 91) (width 0.2) (layer "B.Cu") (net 1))
 (segment (start 142.8 81) (end 147.1 81) (width 0.2) (layer "F.Cu") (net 3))
 (segment (start 147.1 81) (end 148.45 79.65) (width 0.2) (layer "F.Cu") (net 3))
 (segment (start 126 76) (end 133.1 76) (width 0.2) (layer "F.Cu") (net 3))
 (segment (start 148.35 107.65) (end 143.5 112.5) (width 0.2) (layer "F.Cu") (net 3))
 (segment (start 148.45 107.65) (end 148.35 107.65) (width 0.2) (layer "F.Cu") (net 3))
 (segment (start 132.808098 91.81645) (end 132.499 92.125548) (width 0.2) (layer "F.Cu") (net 3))
 (segment (start 143.5 112.5) (end 140 116) (width 0.2) (layer "F.Cu") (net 3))
 (segment (start 138.6329 87) (end 133.81645 91.81645) (width 0.2) (layer "F.Cu") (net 3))
 (segment (start 130.35 137.401) (end 131.949 139) (width 0.2) (layer "F.Cu") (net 3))
 (segment (start 123.699 134.899) (end 118.725548 134.899) (width 0.2) (layer "F.Cu") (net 3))
 (segment (start 130.0152 106.5048) (end 128.87 107.65) (width 0.2) (layer "F.Cu") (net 3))
 (segment (start 116 107.1) (end 115.45 107.65) (width 0.2) (layer "F.Cu") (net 3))
 (segment (start 137.149 138.549) (end 132.175548 138.549) (width 0.2) (layer "F.Cu") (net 3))
 (segment (start 125.501 129.9339) (end 125.501 134.599) (width 0.2) (layer "F.Cu") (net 3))
 (segment (start 125.501 134.599) (end 124.45 135.65) (width 0.2) (layer "F.Cu") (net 3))
 (segment (start 128.87 107.65) (end 115.45 107.65) (width 0.2) (layer "F.Cu") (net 3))
 (segment (start 134 101) (end 138 101) (width 0.2) (layer "F.Cu") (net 3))
 (segment (start 119.401 137.401) (end 130.35 137.401) (width 0.2) (layer "F.Cu") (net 3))
 (segment (start 134.324548 95) (end 138 95) (width 0.2) (layer "F.Cu") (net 3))
 (segment (start 132.8339 141.401) (end 139.599 141.401) (width 0.2) (layer "F.Cu") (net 3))
 (segment (start 132.175548 138.549) (end 131.949 138.775548) (width 0.2) (layer "F.Cu") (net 3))
 (segment (start 117.45 122.65) (end 118.2171 122.65) (width 0.2) (layer "F.Cu") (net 3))
 (segment (start 133.1 76) (end 135.45 73.65) (width 0.2) (layer "F.Cu") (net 3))
 (segment (start 116.45 92.65) (end 116.825452 92.65) (width 0.2) (layer "F.Cu") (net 3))
 (segment (start 118.499 136.499) (end 119.401 137.401) (width 0.2) (layer "F.Cu") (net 3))
 (segment (start 139 116) (end 138 117) (width 0.2) (layer "F.Cu") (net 3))
 (segment (start 137.9 139.3) (end 137.149 138.549) (width 0.2) (layer "F.Cu") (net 3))
 (segment (start 138 101) (end 138 95) (width 0.2) (layer "F.Cu") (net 3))
 (segment (start 118.2171 122.65) (end 125.501 129.9339) (width 0.2) (layer "F.Cu") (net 3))
 (segment (start 118.725548 134.899) (end 118.499 135.125548) (width 0.2) (layer "F.Cu") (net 3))
 (segment (start 115.45 107.65) (end 118.501 110.701) (width 0.2) (layer "F.Cu") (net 3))
 (segment (start 139.599 141.401) (end 148.35 132.65) (width 0.2) (layer "F.Cu") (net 3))
 (segment (start 130.0152 106) (end 130.0152 106.5048) (width 0.2) (layer "F.Cu") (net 3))
 (segment (start 116 106) (end 116 107.1) (width 0.2) (layer "F.Cu") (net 3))
 (segment (start 142.8 81) (end 142.8 86.2) (width 0.2) (layer "F.Cu") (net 3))
 (segment (start 122.45 78.65) (end 123.35 78.65) (width 0.2) (layer "F.Cu") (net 3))
 (segment (start 138 93.1) (end 138.45 92.65) (width 0.2) (layer "F.Cu") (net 3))
 (segment (start 138 117) (end 138 119.2) (width 0.2) (layer "F.Cu") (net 3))
 (segment (start 138 119.2) (end 139.45 120.65) (width 0.2) (layer "F.Cu") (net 3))
 (segment (start 124.45 135.65) (end 123.699 134.899) (width 0.2) (layer "F.Cu") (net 3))
 (segment (start 116.899999 105.100001) (end 116 106) (width 0.2) (layer "F.Cu") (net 3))
 (segment (start 138 101) (end 138 107) (width 0.2) (layer "F.Cu") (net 3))
 (segment (start 132.499 93.174452) (end 134.324548 95) (width 0.2) (layer "F.Cu") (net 3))
 (segment (start 131.949 140.5161) (end 132.8339 141.401) (width 0.2) (layer "F.Cu") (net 3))
 (segment (start 148.45 79.65) (end 147.95 79.65) (width 0.2) (layer "F.Cu") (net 3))
 (segment (start 138 107) (end 143.5 112.5) (width 0.2) (layer "F.Cu") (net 3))
 (segment (start 130.0152 106) (end 130.0152 104.9848) (width 0.2) (layer "F.Cu") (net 3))
 (segment (start 118.501 110.701) (end 118.501 121.599) (width 0.2) (layer "F.Cu") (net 3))
 (segment (start 138 95) (end 138 93.1) (width 0.2) (layer "F.Cu") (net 3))
 (segment (start 130.0152 104.9848) (end 134 101) (width 0.2) (layer "F.Cu") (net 3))
 (segment (start 142.8 86.2) (end 142 87) (width 0.2) (layer "F.Cu") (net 3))
 (segment (start 140 116) (end 139 116) (width 0.2) (layer "F.Cu") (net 3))
 (segment (start 118.499 135.125548) (end 118.499 136.499) (width 0.2) (layer "F.Cu") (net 3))
 (segment (start 131.949 139) (end 131.949 140.5161) (width 0.2) (layer "F.Cu") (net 3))
 (segment (start 133.81645 91.81645) (end 132.808098 91.81645) (width 0.2) (layer "F.Cu") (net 3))
 (segment (start 116.45 92.65) (end 116.899999 93.099999) (width 0.2) (layer "F.Cu") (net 3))
 (segment (start 118.501 121.599) (end 117.45 122.65) (width 0.2) (layer "F.Cu") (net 3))
 (segment (start 142 87) (end 138.6329 87) (width 0.2) (layer "F.Cu") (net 3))
 (segment (start 131.949 138.775548) (end 131.949 139) (width 0.2) (layer "F.Cu") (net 3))
 (segment (start 148.35 132.65) (end 150.45 132.65) (width 0.2) (layer "F.Cu") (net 3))
 (segment (start 123.35 78.65) (end 126 76) (width 0.2) (layer "F.Cu") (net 3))
 (segment (start 132.499 92.125548) (end 132.499 93.174452) (width 0.2) (layer "F.Cu") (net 3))
 (segment (start 116.899999 93.099999) (end 116.899999 105.100001) (width 0.2) (layer "F.Cu") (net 3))
 (segment (start 135.45 73.65) (end 142.8 81) (width 0.2) (layer "F.Cu") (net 3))
 (via (at 116 106) (size 0.6) (drill 0.3) (layers "F.Cu" "B.Cu") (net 3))
 (segment (start 118.370001 106.000001) (end 116 106) (width 0.2) (layer "B.Cu") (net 3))
 (segment (start 143.55 107.65) (end 140 104.1) (width 0.2) (layer "F.Cu") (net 6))
 (segment (start 140 104.1) (end 140 90.9) (width 0.2) (layer "F.Cu") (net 6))
 (segment (start 140 90.9) (end 138.45 89.35) (width 0.2) (layer "F.Cu") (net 6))
 (segment (start 124.15 73.65) (end 122.45 75.35) (width 0.2) (layer "F.Cu") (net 14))
 (segment (start 130.55 73.65) (end 124.15 73.65) (width 0.2) (layer "F.Cu") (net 14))
 (segment (start 116.45 79.75) (end 116.45 89.35) (width 0.2) (layer "F.Cu") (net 8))
 (segment (start 117.55 78.65) (end 116.45 79.75) (width 0.2) (layer "F.Cu") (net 8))
 (segment (start 111.55 92.65) (end 115.45 96.55) (width 0.2) (layer "F.Cu") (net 7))
 (segment (start 115.45 96.55) (end 115.45 104.35) (width 0.2) (layer "F.Cu") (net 7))
 (segment (start 110.55 107.65) (end 117.45 114.55) (width 0.2) (layer "F.Cu") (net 10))
 (segment (start 117.45 114.55) (end 117.45 119.35) (width 0.2) (layer "F.Cu") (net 10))
 (segment (start 133.55 92.65) (end 138.2 88) (width 0.2) (layer "F.Cu") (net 5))
 (segment (start 148 82) (end 150 82) (width 0.2) (layer "F.Cu") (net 5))
 (segment (start 138.2 88) (end 142 88) (width 0.2) (layer "F.Cu") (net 5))
 (segment (start 150 77.9) (end 148.45 76.35) (width 0.2) (layer "F.Cu") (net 5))
 (segment (start 142 88) (end 148 82) (width 0.2) (layer "F.Cu") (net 5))
 (segment (start 150 82) (end 150 77.9) (width 0.2) (layer "F.Cu") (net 5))
 (segment (start 143.55 79.65) (end 135.45 71.55) (width 0.2) (layer "F.Cu") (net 12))
 (segment (start 135.45 71.55) (end 135.45 70.35) (width 0.2) (layer "F.Cu") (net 12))
 (segment (start 113.9 124) (end 116 124) (width 0.2) (layer "F.Cu") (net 9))
 (segment (start 121 126) (end 124 129) (width 0.2) (layer "F.Cu") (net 9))
 (segment (start 118 126) (end 121 126) (width 0.2) (layer "F.Cu") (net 9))
 (segment (start 124 129) (end 124.000001 131.900001) (width 0.2) (layer "F.Cu") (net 9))
 (segment (start 112.55 122.65) (end 113.9 124) (width 0.2) (layer "F.Cu") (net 9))
 (segment (start 116 124) (end 118 126) (width 0.2) (layer "F.Cu") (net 9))
 (segment (start 124.000001 131.900001) (end 124.45 132.35) (width 0.2) (layer "F.Cu") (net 9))
 (segment (start 119.55 135.65) (end 120.9 137) (width 0.2) (layer "F.Cu") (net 11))
 (segment (start 136 138) (end 136 137.9) (width 0.2) (layer "F.Cu") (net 11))
 (segment (start 120.9 137) (end 136.9 137) (width 0.2) (layer "F.Cu") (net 11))
 (segment (start 136.9 137) (end 137.9 136) (width 0.2) (layer "F.Cu") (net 11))
 (segment (start 146 106) (end 147.65 104.35) (width 0.2) (layer "F.Cu") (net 16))
 (segment (start 144 111) (end 146 109) (width 0.2) (layer "F.Cu") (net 16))
 (segment (start 146 109) (end 146 106) (width 0.2) (layer "F.Cu") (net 16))
 (segment (start 147.65 104.35) (end 148.45 104.35) (width 0.2) (layer "F.Cu") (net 16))
 (via (at 144 111) (size 0.6) (drill 0.3) (layers "F.Cu" "B.Cu") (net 16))
 (segment (start 120.370001 111) (end 123 111) (width 0.2) (layer "B.Cu") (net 16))
 (segment (start 123 111) (end 144 111) (width 0.2) (layer "B.Cu") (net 16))
 (segment (start 118.370001 109) (end 120.370001 111) (width 0.2) (layer "B.Cu") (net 16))
 (segment (start 133 139.3) (end 133 141) (width 0.2) (layer "F.Cu") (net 4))
 (segment (start 133 141) (end 138.8 141) (width 0.2) (layer "F.Cu") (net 4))
 (segment (start 138.8 141) (end 150.45 129.35) (width 0.2) (layer "F.Cu") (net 4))
 (segment (start 126 104.965201) (end 127.9848 106.950001) (width 0.2) (layer "F.Cu") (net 15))
 (segment (start 126 104) (end 126 104.965201) (width 0.2) (layer "F.Cu") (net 15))
 (via (at 126 104) (size 0.6) (drill 0.3) (layers "F.Cu" "B.Cu") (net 15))
 (segment (start 123 103.000002) (end 125.000002 103.000002) (width 0.2) (layer "B.Cu") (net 15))
 (segment (start 125.000002 103.000002) (end 126 104) (width 0.2) (layer "B.Cu") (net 15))
 (segment (start 141 123) (end 141 118.9) (width 0.2) (layer "F.Cu") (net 2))
 (segment (start 148 130) (end 141 123) (width 0.2) (layer "F.Cu") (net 2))
 (segment (start 148 130.2) (end 148 130) (width 0.2) (layer "F.Cu") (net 2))
 (segment (start 145.55 132.65) (end 148 130.2) (width 0.2) (layer "F.Cu") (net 2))
 (segment (start 141 118.9) (end 139.45 117.35) (width 0.2) (layer "F.Cu") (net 2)))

